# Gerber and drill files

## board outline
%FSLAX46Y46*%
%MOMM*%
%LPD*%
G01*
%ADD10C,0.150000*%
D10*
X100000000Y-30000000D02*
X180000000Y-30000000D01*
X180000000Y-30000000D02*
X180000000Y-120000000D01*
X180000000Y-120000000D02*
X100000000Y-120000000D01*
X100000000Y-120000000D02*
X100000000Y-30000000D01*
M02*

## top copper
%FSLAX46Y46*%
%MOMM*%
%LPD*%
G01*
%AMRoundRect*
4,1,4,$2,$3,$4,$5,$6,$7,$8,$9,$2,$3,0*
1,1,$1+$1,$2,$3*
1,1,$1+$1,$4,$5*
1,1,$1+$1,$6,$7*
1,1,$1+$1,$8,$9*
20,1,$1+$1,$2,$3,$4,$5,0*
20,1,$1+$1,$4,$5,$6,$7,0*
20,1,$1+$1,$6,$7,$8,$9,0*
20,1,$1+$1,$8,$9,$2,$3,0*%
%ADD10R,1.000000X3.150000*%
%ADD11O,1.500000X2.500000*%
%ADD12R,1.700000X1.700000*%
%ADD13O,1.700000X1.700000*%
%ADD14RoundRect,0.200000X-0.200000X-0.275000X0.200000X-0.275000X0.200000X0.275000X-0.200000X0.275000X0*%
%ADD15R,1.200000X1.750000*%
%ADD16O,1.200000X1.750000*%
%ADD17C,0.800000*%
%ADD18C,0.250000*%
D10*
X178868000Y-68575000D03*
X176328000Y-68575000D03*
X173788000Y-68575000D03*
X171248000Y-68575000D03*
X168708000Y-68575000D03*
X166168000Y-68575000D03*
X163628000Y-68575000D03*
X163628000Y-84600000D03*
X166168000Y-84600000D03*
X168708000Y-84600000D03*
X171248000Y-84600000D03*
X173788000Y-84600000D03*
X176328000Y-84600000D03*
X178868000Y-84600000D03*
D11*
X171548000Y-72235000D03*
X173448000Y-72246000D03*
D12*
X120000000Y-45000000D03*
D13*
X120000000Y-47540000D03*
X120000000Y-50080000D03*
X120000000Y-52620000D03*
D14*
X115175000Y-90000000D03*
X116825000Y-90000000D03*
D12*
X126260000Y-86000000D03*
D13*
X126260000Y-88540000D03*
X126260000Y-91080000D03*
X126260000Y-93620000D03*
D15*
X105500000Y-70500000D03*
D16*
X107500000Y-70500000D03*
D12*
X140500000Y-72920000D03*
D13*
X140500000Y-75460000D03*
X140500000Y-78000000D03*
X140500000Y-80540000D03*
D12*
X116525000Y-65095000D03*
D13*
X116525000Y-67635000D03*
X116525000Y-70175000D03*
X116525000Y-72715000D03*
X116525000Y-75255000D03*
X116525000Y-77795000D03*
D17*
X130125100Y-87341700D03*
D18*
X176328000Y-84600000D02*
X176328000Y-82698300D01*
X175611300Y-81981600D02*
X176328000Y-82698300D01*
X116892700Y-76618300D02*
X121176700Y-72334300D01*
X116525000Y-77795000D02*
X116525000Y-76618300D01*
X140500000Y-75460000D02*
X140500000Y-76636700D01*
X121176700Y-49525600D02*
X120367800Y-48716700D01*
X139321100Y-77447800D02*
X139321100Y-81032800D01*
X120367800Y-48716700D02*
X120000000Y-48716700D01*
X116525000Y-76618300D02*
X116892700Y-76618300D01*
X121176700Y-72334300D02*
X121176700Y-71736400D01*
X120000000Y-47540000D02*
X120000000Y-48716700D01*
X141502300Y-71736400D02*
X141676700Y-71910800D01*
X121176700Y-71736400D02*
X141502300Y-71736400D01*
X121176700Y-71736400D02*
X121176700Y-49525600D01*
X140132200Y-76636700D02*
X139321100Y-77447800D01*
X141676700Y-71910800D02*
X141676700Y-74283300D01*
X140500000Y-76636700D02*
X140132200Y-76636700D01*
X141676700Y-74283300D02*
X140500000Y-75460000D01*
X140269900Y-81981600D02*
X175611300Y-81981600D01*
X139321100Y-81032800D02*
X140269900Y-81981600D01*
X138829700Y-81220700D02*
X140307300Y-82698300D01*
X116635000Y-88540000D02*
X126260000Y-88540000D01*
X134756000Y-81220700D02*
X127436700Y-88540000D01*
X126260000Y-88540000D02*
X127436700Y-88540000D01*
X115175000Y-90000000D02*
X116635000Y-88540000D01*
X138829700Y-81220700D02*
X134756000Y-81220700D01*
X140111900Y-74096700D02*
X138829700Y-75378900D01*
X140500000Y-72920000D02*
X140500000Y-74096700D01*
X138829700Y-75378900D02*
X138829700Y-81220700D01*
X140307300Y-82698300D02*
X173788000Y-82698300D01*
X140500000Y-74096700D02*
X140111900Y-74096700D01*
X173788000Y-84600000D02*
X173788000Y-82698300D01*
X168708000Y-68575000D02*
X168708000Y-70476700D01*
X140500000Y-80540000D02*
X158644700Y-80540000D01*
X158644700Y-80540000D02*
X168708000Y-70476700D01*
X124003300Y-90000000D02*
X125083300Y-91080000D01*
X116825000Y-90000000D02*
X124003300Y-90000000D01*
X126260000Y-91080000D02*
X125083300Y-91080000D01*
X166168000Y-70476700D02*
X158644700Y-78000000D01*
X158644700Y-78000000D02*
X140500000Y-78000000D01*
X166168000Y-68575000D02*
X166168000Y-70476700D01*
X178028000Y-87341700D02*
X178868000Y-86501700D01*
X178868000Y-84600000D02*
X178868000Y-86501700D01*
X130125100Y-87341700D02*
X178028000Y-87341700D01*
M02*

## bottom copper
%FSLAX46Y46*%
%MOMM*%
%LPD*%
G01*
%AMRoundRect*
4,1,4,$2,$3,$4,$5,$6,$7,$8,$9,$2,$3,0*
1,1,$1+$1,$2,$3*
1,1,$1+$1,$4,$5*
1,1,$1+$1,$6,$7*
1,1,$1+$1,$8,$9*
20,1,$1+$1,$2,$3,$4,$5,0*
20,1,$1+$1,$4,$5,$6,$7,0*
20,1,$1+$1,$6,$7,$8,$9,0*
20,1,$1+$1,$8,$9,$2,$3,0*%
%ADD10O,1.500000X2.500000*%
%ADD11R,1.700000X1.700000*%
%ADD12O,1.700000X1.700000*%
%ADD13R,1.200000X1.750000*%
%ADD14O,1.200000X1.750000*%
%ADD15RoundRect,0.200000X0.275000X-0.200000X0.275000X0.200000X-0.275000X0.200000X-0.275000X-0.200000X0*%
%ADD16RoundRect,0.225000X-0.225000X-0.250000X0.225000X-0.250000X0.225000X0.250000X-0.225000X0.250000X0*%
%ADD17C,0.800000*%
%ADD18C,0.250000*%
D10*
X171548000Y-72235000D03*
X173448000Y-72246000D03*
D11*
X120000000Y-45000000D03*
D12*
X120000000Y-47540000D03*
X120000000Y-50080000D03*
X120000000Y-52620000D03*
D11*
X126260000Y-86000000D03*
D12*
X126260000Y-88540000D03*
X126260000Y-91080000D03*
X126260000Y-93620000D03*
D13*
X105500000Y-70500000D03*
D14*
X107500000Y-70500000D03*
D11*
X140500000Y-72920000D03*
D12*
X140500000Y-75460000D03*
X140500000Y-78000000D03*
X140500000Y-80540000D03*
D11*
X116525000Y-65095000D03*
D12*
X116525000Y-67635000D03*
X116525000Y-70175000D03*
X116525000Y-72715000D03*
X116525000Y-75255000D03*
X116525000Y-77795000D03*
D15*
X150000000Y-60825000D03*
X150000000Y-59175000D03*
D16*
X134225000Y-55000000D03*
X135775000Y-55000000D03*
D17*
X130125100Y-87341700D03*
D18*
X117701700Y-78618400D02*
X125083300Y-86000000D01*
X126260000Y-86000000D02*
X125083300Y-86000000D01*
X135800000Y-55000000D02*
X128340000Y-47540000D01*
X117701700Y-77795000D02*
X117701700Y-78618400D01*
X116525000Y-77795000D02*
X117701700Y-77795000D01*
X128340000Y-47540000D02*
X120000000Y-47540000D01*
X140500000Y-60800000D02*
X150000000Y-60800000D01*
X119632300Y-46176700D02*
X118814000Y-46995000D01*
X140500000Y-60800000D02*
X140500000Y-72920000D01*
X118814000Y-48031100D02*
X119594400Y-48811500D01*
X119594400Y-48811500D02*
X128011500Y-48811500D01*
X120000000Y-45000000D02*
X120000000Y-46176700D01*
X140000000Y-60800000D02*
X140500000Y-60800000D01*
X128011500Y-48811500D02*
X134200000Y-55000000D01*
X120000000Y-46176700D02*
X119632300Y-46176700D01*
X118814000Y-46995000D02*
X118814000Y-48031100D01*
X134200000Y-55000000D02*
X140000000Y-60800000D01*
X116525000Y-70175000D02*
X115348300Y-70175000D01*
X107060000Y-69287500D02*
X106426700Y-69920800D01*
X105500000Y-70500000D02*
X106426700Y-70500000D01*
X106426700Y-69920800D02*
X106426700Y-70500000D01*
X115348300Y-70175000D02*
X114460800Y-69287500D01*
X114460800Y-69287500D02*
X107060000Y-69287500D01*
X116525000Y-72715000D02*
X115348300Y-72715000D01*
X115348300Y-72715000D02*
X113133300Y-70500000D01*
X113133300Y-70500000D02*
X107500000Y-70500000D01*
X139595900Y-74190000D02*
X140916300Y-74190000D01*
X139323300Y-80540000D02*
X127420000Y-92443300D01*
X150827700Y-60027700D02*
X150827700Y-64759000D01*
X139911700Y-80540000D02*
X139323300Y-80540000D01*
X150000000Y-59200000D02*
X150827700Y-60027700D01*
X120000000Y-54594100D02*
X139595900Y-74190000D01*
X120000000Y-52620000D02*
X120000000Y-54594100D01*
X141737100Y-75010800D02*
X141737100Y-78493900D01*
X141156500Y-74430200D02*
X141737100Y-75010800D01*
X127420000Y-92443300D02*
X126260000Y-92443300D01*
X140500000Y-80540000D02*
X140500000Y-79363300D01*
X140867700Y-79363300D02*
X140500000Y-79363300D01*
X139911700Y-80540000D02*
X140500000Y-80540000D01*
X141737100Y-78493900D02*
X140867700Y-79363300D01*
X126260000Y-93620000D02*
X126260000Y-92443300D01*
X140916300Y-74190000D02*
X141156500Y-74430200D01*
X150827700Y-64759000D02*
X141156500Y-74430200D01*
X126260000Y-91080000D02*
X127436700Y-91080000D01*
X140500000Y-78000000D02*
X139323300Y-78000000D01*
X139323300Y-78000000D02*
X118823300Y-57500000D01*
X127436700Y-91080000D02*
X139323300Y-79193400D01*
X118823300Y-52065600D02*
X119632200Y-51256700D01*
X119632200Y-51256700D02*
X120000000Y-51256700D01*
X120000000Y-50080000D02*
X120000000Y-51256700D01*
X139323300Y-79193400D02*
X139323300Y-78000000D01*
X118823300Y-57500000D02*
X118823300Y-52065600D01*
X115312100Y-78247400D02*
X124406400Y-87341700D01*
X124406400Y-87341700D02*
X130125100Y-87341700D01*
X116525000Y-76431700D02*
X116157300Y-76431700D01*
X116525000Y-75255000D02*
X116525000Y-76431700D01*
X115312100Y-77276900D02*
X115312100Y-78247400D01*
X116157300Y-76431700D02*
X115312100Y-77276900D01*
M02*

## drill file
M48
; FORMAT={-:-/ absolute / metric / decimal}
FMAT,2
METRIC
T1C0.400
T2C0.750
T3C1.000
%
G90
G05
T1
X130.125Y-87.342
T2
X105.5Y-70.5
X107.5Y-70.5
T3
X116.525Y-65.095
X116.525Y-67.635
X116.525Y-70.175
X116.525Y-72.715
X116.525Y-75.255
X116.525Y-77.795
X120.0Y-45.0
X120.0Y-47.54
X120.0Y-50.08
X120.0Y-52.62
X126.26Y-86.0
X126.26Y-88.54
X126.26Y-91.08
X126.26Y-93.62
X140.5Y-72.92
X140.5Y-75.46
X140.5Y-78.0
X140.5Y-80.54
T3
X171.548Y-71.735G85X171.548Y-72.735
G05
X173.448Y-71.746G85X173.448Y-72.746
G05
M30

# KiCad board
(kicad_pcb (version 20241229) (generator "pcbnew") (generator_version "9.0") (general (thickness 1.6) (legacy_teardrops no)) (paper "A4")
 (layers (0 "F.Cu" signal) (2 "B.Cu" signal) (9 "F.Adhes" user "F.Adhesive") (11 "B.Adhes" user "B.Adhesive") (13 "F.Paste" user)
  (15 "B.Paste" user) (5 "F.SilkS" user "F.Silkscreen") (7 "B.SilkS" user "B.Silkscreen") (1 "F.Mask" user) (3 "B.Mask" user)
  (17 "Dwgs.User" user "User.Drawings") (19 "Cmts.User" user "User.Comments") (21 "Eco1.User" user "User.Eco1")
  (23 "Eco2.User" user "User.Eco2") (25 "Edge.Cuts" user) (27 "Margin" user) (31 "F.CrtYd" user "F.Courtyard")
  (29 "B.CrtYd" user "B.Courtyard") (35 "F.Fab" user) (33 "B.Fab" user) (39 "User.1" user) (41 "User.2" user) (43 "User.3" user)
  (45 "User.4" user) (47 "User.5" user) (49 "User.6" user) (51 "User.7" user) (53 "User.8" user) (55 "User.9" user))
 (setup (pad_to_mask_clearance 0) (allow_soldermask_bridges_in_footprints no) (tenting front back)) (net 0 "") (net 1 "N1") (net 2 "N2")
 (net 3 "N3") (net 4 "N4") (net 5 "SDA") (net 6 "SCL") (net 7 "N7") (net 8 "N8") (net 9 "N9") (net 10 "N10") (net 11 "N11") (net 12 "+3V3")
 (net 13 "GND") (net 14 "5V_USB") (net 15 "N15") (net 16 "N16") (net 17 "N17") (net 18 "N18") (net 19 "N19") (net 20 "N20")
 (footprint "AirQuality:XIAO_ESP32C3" (layer "F.Cu") (at 169.448 77.175 -90)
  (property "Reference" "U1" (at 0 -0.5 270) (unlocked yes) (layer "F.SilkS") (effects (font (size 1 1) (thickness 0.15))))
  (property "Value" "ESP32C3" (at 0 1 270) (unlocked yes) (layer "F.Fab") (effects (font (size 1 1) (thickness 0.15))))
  (pad "1" smd rect (at -8.6 -9.42 270) (size 3.15 1) (layers "F.Cu" "F.Mask" "F.Paste") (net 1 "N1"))
  (pad "2" smd rect (at -8.6 -6.88 270) (size 3.15 1) (layers "F.Cu" "F.Mask" "F.Paste") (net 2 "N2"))
  (pad "3" smd rect (at -8.6 -4.34 270) (size 3.15 1) (layers "F.Cu" "F.Mask" "F.Paste") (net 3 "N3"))
  (pad "4" smd rect (at -8.6 -1.8 270) (size 3.15 1) (layers "F.Cu" "F.Mask" "F.Paste") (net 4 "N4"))
  (pad "5" smd rect (at -8.6 0.74 270) (size 3.15 1) (layers "F.Cu" "F.Mask" "F.Paste") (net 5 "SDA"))
  (pad "6" smd rect (at -8.6 3.28 270) (size 3.15 1) (layers "F.Cu" "F.Mask" "F.Paste") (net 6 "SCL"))
  (pad "7" smd rect (at -8.6 5.82 270) (size 3.15 1) (layers "F.Cu" "F.Mask" "F.Paste") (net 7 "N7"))
  (pad "8" smd rect (at 7.425 5.82 270) (size 3.15 1) (layers "F.Cu" "F.Mask" "F.Paste") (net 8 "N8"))
  (pad "9" smd rect (at 7.425 3.28 270) (size 3.15 1) (layers "F.Cu" "F.Mask" "F.Paste") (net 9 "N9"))
  (pad "10" smd rect (at 7.425 0.74 270) (size 3.15 1) (layers "F.Cu" "F.Mask" "F.Paste") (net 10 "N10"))
  (pad "11" smd rect (at 7.425 -1.8 270) (size 3.15 1) (layers "F.Cu" "F.Mask" "F.Paste") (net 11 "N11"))
  (pad "12" smd rect (at 7.425 -4.34 270) (size 3.15 1) (layers "F.Cu" "F.Mask" "F.Paste") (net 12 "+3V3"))
  (pad "13" smd rect (at 7.425 -6.88 270) (size 3.15 1) (layers "F.Cu" "F.Mask" "F.Paste") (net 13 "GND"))
  (pad "14" smd rect (at 7.425 -9.42 270) (size 3.15 1) (layers "F.Cu" "F.Mask" "F.Paste") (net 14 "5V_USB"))
  (pad "B+" thru_hole oval (at -4.94 -2.1 270) (size 2.5 1.5) (drill oval 2 1) (layers "*.Cu" "*.Mask") (remove_unused_layers no)
   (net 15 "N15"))
  (pad "B-" thru_hole oval (at -4.929 -4 270) (size 2.5 1.5) (drill oval 2 1) (layers "*.Cu" "*.Mask") (remove_unused_layers no)
   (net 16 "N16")))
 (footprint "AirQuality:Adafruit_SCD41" (layer "F.Cu") (at 120 45)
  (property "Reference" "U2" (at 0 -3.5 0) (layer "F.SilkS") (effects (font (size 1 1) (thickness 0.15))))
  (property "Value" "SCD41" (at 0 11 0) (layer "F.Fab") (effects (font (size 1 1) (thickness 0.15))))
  (pad "1" thru_hole rect (at 0 0) (size 1.7 1.7) (drill 1) (layers "*.Cu" "*.Mask") (remove_unused_layers no) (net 12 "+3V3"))
  (pad "2" thru_hole oval (at 0 2.54) (size 1.7 1.7) (drill 1) (layers "*.Cu" "*.Mask") (remove_unused_layers no) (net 13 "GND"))
  (pad "3" thru_hole oval (at 0 5.08) (size 1.7 1.7) (drill 1) (layers "*.Cu" "*.Mask") (remove_unused_layers no) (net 6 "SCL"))
  (pad "4" thru_hole oval (at 0 7.62) (size 1.7 1.7) (drill 1) (layers "*.Cu" "*.Mask") (remove_unused_layers no) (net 5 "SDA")))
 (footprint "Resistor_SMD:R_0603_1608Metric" (layer "F.Cu") (at 116 90)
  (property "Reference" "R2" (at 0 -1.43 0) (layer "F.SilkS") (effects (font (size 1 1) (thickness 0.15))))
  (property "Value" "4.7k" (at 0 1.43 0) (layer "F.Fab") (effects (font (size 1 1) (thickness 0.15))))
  (pad "1" smd roundrect (at -0.825 0) (size 0.8 0.95) (layers "F.Cu" "F.Mask" "F.Paste") (roundrect_rratio 0.25) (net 12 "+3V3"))
  (pad "2" smd roundrect (at 0.825 0) (size 0.8 0.95) (layers "F.Cu" "F.Mask" "F.Paste") (roundrect_rratio 0.25) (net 6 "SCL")))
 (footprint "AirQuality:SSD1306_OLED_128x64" (layer "F.Cu") (at 126.26 86)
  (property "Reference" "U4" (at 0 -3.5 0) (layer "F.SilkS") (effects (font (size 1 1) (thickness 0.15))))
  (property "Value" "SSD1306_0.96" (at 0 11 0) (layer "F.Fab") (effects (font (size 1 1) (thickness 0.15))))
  (pad "1" thru_hole rect (at 0 0) (size 1.7 1.7) (drill 1) (layers "*.Cu" "*.Mask") (remove_unused_layers no) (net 13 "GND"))
  (pad "2" thru_hole oval (at 0 2.54) (size 1.7 1.7) (drill 1) (layers "*.Cu" "*.Mask") (remove_unused_layers no) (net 12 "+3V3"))
  (pad "3" thru_hole oval (at 0 5.08) (size 1.7 1.7) (drill 1) (layers "*.Cu" "*.Mask") (remove_unused_layers no) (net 6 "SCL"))
  (pad "4" thru_hole oval (at 0 7.62) (size 1.7 1.7) (drill 1) (layers "*.Cu" "*.Mask") (remove_unused_layers no) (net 5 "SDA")))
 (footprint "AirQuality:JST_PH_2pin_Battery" (layer "F.Cu") (at 105.5 70.5)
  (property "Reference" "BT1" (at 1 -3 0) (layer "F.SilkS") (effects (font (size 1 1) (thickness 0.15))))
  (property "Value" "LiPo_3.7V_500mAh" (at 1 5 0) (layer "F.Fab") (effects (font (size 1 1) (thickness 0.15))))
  (pad "1" thru_hole rect (at 0 0) (size 1.2 1.75) (drill 0.75) (layers "*.Cu" "*.Mask") (remove_unused_layers no) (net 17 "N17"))
  (pad "2" thru_hole oval (at 2 0) (size 1.2 1.75) (drill 0.75) (layers "*.Cu" "*.Mask") (remove_unused_layers no) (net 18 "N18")))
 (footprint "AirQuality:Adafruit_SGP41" (layer "F.Cu") (at 140.5 72.92)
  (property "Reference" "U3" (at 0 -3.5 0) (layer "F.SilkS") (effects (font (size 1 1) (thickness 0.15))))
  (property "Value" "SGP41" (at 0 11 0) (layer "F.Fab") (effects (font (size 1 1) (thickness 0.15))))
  (pad "1" thru_hole rect (at 0 0) (size 1.7 1.7) (drill 1) (layers "*.Cu" "*.Mask") (remove_unused_layers no) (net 12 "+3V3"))
  (pad "2" thru_hole oval (at 0 2.54) (size 1.7 1.7) (drill 1) (layers "*.Cu" "*.Mask") (remove_unused_layers no) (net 13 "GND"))
  (pad "3" thru_hole oval (at 0 5.08) (size 1.7 1.7) (drill 1) (layers "*.Cu" "*.Mask") (remove_unused_layers no) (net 6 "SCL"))
  (pad "4" thru_hole oval (at 0 7.62) (size 1.7 1.7) (drill 1) (layers "*.Cu" "*.Mask") (remove_unused_layers no) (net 5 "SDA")))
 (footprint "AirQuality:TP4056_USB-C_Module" (layer "F.Cu") (at 116.525 65.095)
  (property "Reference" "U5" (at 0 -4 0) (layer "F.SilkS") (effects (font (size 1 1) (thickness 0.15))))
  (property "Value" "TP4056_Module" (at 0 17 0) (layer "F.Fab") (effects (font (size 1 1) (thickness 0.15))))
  (pad "1" thru_hole rect (at 0 0) (size 1.7 1.7) (drill 1) (layers "*.Cu" "*.Mask") (remove_unused_layers no) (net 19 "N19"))
  (pad "2" thru_hole oval (at 0 2.54) (size 1.7 1.7) (drill 1) (layers "*.Cu" "*.Mask") (remove_unused_layers no) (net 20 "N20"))
  (pad "3" thru_hole oval (at 0 5.08) (size 1.7 1.7) (drill 1) (layers "*.Cu" "*.Mask") (remove_unused_layers no) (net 17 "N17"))
  (pad "4" thru_hole oval (at 0 7.62) (size 1.7 1.7) (drill 1) (layers "*.Cu" "*.Mask") (remove_unused_layers no) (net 18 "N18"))
  (pad "5" thru_hole oval (at 0 10.16) (size 1.7 1.7) (drill 1) (layers "*.Cu" "*.Mask") (remove_unused_layers no) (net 14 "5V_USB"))
  (pad "6" thru_hole oval (at 0 12.7) (size 1.7 1.7) (drill 1) (layers "*.Cu" "*.Mask") (remove_unused_layers no) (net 13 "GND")))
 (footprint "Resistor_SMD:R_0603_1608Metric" (layer "B.Cu") (at 150 60 90)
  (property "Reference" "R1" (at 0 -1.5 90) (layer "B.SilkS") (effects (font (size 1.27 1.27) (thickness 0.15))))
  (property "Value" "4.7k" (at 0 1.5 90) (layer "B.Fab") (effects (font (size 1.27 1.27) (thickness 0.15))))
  (pad "1" smd roundrect (at -0.825 0 90) (size 0.8 0.95) (layers "B.Cu" "B.Mask" "B.Paste") (roundrect_rratio 0.25) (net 12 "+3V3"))
  (pad "2" smd roundrect (at 0.825 0 90) (size 0.8 0.95) (layers "B.Cu" "B.Mask" "B.Paste") (roundrect_rratio 0.25) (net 5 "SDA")))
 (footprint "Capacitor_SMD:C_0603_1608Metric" (layer "B.Cu") (at 135 55)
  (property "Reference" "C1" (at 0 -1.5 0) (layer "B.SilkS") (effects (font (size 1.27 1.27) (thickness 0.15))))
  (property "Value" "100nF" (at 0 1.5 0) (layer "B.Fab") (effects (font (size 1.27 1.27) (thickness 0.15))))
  (pad "1" smd roundrect (at -0.775 0) (size 0.9 0.95) (layers "B.Cu" "B.Mask" "B.Paste") (roundrect_rratio 0.25) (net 12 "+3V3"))
  (pad "2" smd roundrect (at 0.775 0) (size 0.9 0.95) (layers "B.Cu" "B.Mask" "B.Paste") (roundrect_rratio 0.25) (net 13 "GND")))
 (gr_line (start 100 30) (end 180 30) (stroke (width 0.15) (type solid)) (layer "Edge.Cuts"))
 (gr_line (start 180 30) (end 180 120) (stroke (width 0.15) (type solid)) (layer "Edge.Cuts"))
 (gr_line (start 180 120) (end 100 120) (stroke (width 0.15) (type solid)) (layer "Edge.Cuts"))
 (gr_line (start 100 120) (end 100 30) (stroke (width 0.15) (type solid)) (layer "Edge.Cuts"))
 (segment (start 176.328 84.6) (end 176.328 82.6983) (width 0.25) (layer "F.Cu") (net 13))
 (segment (start 175.6113 81.9816) (end 176.328 82.6983) (width 0.25) (layer "F.Cu") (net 13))
 (segment (start 116.8927 76.6183) (end 121.1767 72.3343) (width 0.25) (layer "F.Cu") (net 13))
 (segment (start 116.525 77.795) (end 116.525 76.6183) (width 0.25) (layer "F.Cu") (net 13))
 (segment (start 140.5 75.46) (end 140.5 76.6367) (width 0.25) (layer "F.Cu") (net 13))
 (segment (start 121.1767 49.5256) (end 120.3678 48.7167) (width 0.25) (layer "F.Cu") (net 13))
 (segment (start 139.3211 77.4478) (end 139.3211 81.0328) (width 0.25) (layer "F.Cu") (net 13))
 (segment (start 120.3678 48.7167) (end 120 48.7167) (width 0.25) (layer "F.Cu") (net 13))
 (segment (start 116.525 76.6183) (end 116.8927 76.6183) (width 0.25) (layer "F.Cu") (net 13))
 (segment (start 121.1767 72.3343) (end 121.1767 71.7364) (width 0.25) (layer "F.Cu") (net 13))
 (segment (start 120 47.54) (end 120 48.7167) (width 0.25) (layer "F.Cu") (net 13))
 (segment (start 141.5023 71.7364) (end 141.6767 71.9108) (width 0.25) (layer "F.Cu") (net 13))
 (segment (start 121.1767 71.7364) (end 141.5023 71.7364) (width 0.25) (layer "F.Cu") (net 13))
 (segment (start 121.1767 71.7364) (end 121.1767 49.5256) (width 0.25) (layer "F.Cu") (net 13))
 (segment (start 140.1322 76.6367) (end 139.3211 77.4478) (width 0.25) (layer "F.Cu") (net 13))
 (segment (start 141.6767 71.9108) (end 141.6767 74.2833) (width 0.25) (layer "F.Cu") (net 13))
 (segment (start 140.5 76.6367) (end 140.1322 76.6367) (width 0.25) (layer "F.Cu") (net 13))
 (segment (start 141.6767 74.2833) (end 140.5 75.46) (width 0.25) (layer "F.Cu") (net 13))
 (segment (start 140.2699 81.9816) (end 175.6113 81.9816) (width 0.25) (layer "F.Cu") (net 13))
 (segment (start 139.3211 81.0328) (end 140.2699 81.9816) (width 0.25) (layer "F.Cu") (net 13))
 (segment (start 117.7017 78.6184) (end 125.0833 86) (width 0.25) (layer "B.Cu") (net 13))
 (segment (start 126.26 86) (end 125.0833 86) (width 0.25) (layer "B.Cu") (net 13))
 (segment (start 135.8 55) (end 128.34 47.54) (width 0.25) (layer "B.Cu") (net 13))
 (segment (start 117.7017 77.795) (end 117.7017 78.6184) (width 0.25) (layer "B.Cu") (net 13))
 (segment (start 116.525 77.795) (end 117.7017 77.795) (width 0.25) (layer "B.Cu") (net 13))
 (segment (start 128.34 47.54) (end 120 47.54) (width 0.25) (layer "B.Cu") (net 13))
 (segment (start 138.8297 81.2207) (end 140.3073 82.6983) (width 0.25) (layer "F.Cu") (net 12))
 (segment (start 116.635 88.54) (end 126.26 88.54) (width 0.25) (layer "F.Cu") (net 12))
 (segment (start 134.756 81.2207) (end 127.4367 88.54) (width 0.25) (layer "F.Cu") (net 12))
 (segment (start 126.26 88.54) (end 127.4367 88.54) (width 0.25) (layer "F.Cu") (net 12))
 (segment (start 115.175 90) (end 116.635 88.54) (width 0.25) (layer "F.Cu") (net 12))
 (segment (start 138.8297 81.2207) (end 134.756 81.2207) (width 0.25) (layer "F.Cu") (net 12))
 (segment (start 140.1119 74.0967) (end 138.8297 75.3789) (width 0.25) (layer "F.Cu") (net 12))
 (segment (start 140.5 72.92) (end 140.5 74.0967) (width 0.25) (layer "F.Cu") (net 12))
 (segment (start 138.8297 75.3789) (end 138.8297 81.2207) (width 0.25) (layer "F.Cu") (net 12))
 (segment (start 140.3073 82.6983) (end 173.788 82.6983) (width 0.25) (layer "F.Cu") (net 12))
 (segment (start 140.5 74.0967) (end 140.1119 74.0967) (width 0.25) (layer "F.Cu") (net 12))
 (segment (start 173.788 84.6) (end 173.788 82.6983) (width 0.25) (layer "F.Cu") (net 12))
 (segment (start 140.5 60.8) (end 150 60.8) (width 0.25) (layer "B.Cu") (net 12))
 (segment (start 119.6323 46.1767) (end 118.814 46.995) (width 0.25) (layer "B.Cu") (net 12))
 (segment (start 140.5 60.8) (end 140.5 72.92) (width 0.25) (layer "B.Cu") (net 12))
 (segment (start 118.814 48.0311) (end 119.5944 48.8115) (width 0.25) (layer "B.Cu") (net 12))
 (segment (start 119.5944 48.8115) (end 128.0115 48.8115) (width 0.25) (layer "B.Cu") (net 12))
 (segment (start 120 45) (end 120 46.1767) (width 0.25) (layer "B.Cu") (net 12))
 (segment (start 140 60.8) (end 140.5 60.8) (width 0.25) (layer "B.Cu") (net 12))
 (segment (start 128.0115 48.8115) (end 134.2 55) (width 0.25) (layer "B.Cu") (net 12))
 (segment (start 120 46.1767) (end 119.6323 46.1767) (width 0.25) (layer "B.Cu") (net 12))
 (segment (start 118.814 46.995) (end 118.814 48.0311) (width 0.25) (layer "B.Cu") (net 12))
 (segment (start 134.2 55) (end 140 60.8) (width 0.25) (layer "B.Cu") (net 12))
 (segment (start 116.525 70.175) (end 115.3483 70.175) (width 0.25) (layer "B.Cu") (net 17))
 (segment (start 107.06 69.2875) (end 106.4267 69.9208) (width 0.25) (layer "B.Cu") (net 17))
 (segment (start 105.5 70.5) (end 106.4267 70.5) (width 0.25) (layer "B.Cu") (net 17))
 (segment (start 106.4267 69.9208) (end 106.4267 70.5) (width 0.25) (layer "B.Cu") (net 17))
 (segment (start 115.3483 70.175) (end 114.4608 69.2875) (width 0.25) (layer "B.Cu") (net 17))
 (segment (start 114.4608 69.2875) (end 107.06 69.2875) (width 0.25) (layer "B.Cu") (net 17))
 (segment (start 116.525 72.715) (end 115.3483 72.715) (width 0.25) (layer "B.Cu") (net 18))
 (segment (start 115.3483 72.715) (end 113.1333 70.5) (width 0.25) (layer "B.Cu") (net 18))
 (segment (start 113.1333 70.5) (end 107.5 70.5) (width 0.25) (layer "B.Cu") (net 18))
 (segment (start 168.708 68.575) (end 168.708 70.4767) (width 0.25) (layer "F.Cu") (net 5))
 (segment (start 140.5 80.54) (end 158.6447 80.54) (width 0.25) (layer "F.Cu") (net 5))
 (segment (start 158.6447 80.54) (end 168.708 70.4767) (width 0.25) (layer "F.Cu") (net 5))
 (segment (start 139.5959 74.19) (end 140.9163 74.19) (width 0.25) (layer "B.Cu") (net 5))
 (segment (start 139.3233 80.54) (end 127.42 92.4433) (width 0.25) (layer "B.Cu") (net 5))
 (segment (start 150.8277 60.0277) (end 150.8277 64.759) (width 0.25) (layer "B.Cu") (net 5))
 (segment (start 139.9117 80.54) (end 139.3233 80.54) (width 0.25) (layer "B.Cu") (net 5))
 (segment (start 150 59.2) (end 150.8277 60.0277) (width 0.25) (layer "B.Cu") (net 5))
 (segment (start 120 54.5941) (end 139.5959 74.19) (width 0.25) (layer "B.Cu") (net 5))
 (segment (start 120 52.62) (end 120 54.5941) (width 0.25) (layer "B.Cu") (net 5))
 (segment (start 141.7371 75.0108) (end 141.7371 78.4939) (width 0.25) (layer "B.Cu") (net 5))
 (segment (start 141.1565 74.4302) (end 141.7371 75.0108) (width 0.25) (layer "B.Cu") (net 5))
 (segment (start 127.42 92.4433) (end 126.26 92.4433) (width 0.25) (layer "B.Cu") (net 5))
 (segment (start 140.5 80.54) (end 140.5 79.3633) (width 0.25) (layer "B.Cu") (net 5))
 (segment (start 140.8677 79.3633) (end 140.5 79.3633) (width 0.25) (layer "B.Cu") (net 5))
 (segment (start 139.9117 80.54) (end 140.5 80.54) (width 0.25) (layer "B.Cu") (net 5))
 (segment (start 141.7371 78.4939) (end 140.8677 79.3633) (width 0.25) (layer "B.Cu") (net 5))
 (segment (start 126.26 93.62) (end 126.26 92.4433) (width 0.25) (layer "B.Cu") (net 5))
 (segment (start 140.9163 74.19) (end 141.1565 74.4302) (width 0.25) (layer "B.Cu") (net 5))
 (segment (start 150.8277 64.759) (end 141.1565 74.4302) (width 0.25) (layer "B.Cu") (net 5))
 (segment (start 124.0033 90) (end 125.0833 91.08) (width 0.25) (layer "F.Cu") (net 6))
 (segment (start 116.825 90) (end 124.0033 90) (width 0.25) (layer "F.Cu") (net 6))
 (segment (start 126.26 91.08) (end 125.0833 91.08) (width 0.25) (layer "F.Cu") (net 6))
 (segment (start 166.168 70.4767) (end 158.6447 78) (width 0.25) (layer "F.Cu") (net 6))
 (segment (start 158.6447 78) (end 140.5 78) (width 0.25) (layer "F.Cu") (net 6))
 (segment (start 166.168 68.575) (end 166.168 70.4767) (width 0.25) (layer "F.Cu") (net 6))
 (segment (start 126.26 91.08) (end 127.4367 91.08) (width 0.25) (layer "B.Cu") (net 6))
 (segment (start 140.5 78) (end 139.3233 78) (width 0.25) (layer "B.Cu") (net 6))
 (segment (start 139.3233 78) (end 118.8233 57.5) (width 0.25) (layer "B.Cu") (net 6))
 (segment (start 127.4367 91.08) (end 139.3233 79.1934) (width 0.25) (layer "B.Cu") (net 6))
 (segment (start 118.8233 52.0656) (end 119.6322 51.2567) (width 0.25) (layer "B.Cu") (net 6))
 (segment (start 119.6322 51.2567) (end 120 51.2567) (width 0.25) (layer "B.Cu") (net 6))
 (segment (start 120 50.08) (end 120 51.2567) (width 0.25) (layer "B.Cu") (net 6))
 (segment (start 139.3233 79.1934) (end 139.3233 78) (width 0.25) (layer "B.Cu") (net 6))
 (segment (start 118.8233 57.5) (end 118.8233 52.0656) (width 0.25) (layer "B.Cu") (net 6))
 (segment (start 178.028 87.3417) (end 178.868 86.5017) (width 0.25) (layer "F.Cu") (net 14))
 (segment (start 178.868 84.6) (end 178.868 86.5017) (width 0.25) (layer "F.Cu") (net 14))
 (segment (start 130.1251 87.3417) (end 178.028 87.3417) (width 0.25) (layer "F.Cu") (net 14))
 (via (at 130.1251 87.3417) (size 0.8) (drill 0.4) (layers "F.Cu" "B.Cu") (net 14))
 (segment (start 115.3121 78.2474) (end 124.4064 87.3417) (width 0.25) (layer "B.Cu") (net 14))
 (segment (start 124.4064 87.3417) (end 130.1251 87.3417) (width 0.25) (layer "B.Cu") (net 14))
 (segment (start 116.525 76.4317) (end 116.1573 76.4317) (width 0.25) (layer "B.Cu") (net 14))
 (segment (start 116.525 75.255) (end 116.525 76.4317) (width 0.25) (layer "B.Cu") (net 14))
 (segment (start 115.3121 77.2769) (end 115.3121 78.2474) (width 0.25) (layer "B.Cu") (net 14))
 (segment (start 116.1573 76.4317) (end 115.3121 77.2769) (width 0.25) (layer "B.Cu") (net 14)))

